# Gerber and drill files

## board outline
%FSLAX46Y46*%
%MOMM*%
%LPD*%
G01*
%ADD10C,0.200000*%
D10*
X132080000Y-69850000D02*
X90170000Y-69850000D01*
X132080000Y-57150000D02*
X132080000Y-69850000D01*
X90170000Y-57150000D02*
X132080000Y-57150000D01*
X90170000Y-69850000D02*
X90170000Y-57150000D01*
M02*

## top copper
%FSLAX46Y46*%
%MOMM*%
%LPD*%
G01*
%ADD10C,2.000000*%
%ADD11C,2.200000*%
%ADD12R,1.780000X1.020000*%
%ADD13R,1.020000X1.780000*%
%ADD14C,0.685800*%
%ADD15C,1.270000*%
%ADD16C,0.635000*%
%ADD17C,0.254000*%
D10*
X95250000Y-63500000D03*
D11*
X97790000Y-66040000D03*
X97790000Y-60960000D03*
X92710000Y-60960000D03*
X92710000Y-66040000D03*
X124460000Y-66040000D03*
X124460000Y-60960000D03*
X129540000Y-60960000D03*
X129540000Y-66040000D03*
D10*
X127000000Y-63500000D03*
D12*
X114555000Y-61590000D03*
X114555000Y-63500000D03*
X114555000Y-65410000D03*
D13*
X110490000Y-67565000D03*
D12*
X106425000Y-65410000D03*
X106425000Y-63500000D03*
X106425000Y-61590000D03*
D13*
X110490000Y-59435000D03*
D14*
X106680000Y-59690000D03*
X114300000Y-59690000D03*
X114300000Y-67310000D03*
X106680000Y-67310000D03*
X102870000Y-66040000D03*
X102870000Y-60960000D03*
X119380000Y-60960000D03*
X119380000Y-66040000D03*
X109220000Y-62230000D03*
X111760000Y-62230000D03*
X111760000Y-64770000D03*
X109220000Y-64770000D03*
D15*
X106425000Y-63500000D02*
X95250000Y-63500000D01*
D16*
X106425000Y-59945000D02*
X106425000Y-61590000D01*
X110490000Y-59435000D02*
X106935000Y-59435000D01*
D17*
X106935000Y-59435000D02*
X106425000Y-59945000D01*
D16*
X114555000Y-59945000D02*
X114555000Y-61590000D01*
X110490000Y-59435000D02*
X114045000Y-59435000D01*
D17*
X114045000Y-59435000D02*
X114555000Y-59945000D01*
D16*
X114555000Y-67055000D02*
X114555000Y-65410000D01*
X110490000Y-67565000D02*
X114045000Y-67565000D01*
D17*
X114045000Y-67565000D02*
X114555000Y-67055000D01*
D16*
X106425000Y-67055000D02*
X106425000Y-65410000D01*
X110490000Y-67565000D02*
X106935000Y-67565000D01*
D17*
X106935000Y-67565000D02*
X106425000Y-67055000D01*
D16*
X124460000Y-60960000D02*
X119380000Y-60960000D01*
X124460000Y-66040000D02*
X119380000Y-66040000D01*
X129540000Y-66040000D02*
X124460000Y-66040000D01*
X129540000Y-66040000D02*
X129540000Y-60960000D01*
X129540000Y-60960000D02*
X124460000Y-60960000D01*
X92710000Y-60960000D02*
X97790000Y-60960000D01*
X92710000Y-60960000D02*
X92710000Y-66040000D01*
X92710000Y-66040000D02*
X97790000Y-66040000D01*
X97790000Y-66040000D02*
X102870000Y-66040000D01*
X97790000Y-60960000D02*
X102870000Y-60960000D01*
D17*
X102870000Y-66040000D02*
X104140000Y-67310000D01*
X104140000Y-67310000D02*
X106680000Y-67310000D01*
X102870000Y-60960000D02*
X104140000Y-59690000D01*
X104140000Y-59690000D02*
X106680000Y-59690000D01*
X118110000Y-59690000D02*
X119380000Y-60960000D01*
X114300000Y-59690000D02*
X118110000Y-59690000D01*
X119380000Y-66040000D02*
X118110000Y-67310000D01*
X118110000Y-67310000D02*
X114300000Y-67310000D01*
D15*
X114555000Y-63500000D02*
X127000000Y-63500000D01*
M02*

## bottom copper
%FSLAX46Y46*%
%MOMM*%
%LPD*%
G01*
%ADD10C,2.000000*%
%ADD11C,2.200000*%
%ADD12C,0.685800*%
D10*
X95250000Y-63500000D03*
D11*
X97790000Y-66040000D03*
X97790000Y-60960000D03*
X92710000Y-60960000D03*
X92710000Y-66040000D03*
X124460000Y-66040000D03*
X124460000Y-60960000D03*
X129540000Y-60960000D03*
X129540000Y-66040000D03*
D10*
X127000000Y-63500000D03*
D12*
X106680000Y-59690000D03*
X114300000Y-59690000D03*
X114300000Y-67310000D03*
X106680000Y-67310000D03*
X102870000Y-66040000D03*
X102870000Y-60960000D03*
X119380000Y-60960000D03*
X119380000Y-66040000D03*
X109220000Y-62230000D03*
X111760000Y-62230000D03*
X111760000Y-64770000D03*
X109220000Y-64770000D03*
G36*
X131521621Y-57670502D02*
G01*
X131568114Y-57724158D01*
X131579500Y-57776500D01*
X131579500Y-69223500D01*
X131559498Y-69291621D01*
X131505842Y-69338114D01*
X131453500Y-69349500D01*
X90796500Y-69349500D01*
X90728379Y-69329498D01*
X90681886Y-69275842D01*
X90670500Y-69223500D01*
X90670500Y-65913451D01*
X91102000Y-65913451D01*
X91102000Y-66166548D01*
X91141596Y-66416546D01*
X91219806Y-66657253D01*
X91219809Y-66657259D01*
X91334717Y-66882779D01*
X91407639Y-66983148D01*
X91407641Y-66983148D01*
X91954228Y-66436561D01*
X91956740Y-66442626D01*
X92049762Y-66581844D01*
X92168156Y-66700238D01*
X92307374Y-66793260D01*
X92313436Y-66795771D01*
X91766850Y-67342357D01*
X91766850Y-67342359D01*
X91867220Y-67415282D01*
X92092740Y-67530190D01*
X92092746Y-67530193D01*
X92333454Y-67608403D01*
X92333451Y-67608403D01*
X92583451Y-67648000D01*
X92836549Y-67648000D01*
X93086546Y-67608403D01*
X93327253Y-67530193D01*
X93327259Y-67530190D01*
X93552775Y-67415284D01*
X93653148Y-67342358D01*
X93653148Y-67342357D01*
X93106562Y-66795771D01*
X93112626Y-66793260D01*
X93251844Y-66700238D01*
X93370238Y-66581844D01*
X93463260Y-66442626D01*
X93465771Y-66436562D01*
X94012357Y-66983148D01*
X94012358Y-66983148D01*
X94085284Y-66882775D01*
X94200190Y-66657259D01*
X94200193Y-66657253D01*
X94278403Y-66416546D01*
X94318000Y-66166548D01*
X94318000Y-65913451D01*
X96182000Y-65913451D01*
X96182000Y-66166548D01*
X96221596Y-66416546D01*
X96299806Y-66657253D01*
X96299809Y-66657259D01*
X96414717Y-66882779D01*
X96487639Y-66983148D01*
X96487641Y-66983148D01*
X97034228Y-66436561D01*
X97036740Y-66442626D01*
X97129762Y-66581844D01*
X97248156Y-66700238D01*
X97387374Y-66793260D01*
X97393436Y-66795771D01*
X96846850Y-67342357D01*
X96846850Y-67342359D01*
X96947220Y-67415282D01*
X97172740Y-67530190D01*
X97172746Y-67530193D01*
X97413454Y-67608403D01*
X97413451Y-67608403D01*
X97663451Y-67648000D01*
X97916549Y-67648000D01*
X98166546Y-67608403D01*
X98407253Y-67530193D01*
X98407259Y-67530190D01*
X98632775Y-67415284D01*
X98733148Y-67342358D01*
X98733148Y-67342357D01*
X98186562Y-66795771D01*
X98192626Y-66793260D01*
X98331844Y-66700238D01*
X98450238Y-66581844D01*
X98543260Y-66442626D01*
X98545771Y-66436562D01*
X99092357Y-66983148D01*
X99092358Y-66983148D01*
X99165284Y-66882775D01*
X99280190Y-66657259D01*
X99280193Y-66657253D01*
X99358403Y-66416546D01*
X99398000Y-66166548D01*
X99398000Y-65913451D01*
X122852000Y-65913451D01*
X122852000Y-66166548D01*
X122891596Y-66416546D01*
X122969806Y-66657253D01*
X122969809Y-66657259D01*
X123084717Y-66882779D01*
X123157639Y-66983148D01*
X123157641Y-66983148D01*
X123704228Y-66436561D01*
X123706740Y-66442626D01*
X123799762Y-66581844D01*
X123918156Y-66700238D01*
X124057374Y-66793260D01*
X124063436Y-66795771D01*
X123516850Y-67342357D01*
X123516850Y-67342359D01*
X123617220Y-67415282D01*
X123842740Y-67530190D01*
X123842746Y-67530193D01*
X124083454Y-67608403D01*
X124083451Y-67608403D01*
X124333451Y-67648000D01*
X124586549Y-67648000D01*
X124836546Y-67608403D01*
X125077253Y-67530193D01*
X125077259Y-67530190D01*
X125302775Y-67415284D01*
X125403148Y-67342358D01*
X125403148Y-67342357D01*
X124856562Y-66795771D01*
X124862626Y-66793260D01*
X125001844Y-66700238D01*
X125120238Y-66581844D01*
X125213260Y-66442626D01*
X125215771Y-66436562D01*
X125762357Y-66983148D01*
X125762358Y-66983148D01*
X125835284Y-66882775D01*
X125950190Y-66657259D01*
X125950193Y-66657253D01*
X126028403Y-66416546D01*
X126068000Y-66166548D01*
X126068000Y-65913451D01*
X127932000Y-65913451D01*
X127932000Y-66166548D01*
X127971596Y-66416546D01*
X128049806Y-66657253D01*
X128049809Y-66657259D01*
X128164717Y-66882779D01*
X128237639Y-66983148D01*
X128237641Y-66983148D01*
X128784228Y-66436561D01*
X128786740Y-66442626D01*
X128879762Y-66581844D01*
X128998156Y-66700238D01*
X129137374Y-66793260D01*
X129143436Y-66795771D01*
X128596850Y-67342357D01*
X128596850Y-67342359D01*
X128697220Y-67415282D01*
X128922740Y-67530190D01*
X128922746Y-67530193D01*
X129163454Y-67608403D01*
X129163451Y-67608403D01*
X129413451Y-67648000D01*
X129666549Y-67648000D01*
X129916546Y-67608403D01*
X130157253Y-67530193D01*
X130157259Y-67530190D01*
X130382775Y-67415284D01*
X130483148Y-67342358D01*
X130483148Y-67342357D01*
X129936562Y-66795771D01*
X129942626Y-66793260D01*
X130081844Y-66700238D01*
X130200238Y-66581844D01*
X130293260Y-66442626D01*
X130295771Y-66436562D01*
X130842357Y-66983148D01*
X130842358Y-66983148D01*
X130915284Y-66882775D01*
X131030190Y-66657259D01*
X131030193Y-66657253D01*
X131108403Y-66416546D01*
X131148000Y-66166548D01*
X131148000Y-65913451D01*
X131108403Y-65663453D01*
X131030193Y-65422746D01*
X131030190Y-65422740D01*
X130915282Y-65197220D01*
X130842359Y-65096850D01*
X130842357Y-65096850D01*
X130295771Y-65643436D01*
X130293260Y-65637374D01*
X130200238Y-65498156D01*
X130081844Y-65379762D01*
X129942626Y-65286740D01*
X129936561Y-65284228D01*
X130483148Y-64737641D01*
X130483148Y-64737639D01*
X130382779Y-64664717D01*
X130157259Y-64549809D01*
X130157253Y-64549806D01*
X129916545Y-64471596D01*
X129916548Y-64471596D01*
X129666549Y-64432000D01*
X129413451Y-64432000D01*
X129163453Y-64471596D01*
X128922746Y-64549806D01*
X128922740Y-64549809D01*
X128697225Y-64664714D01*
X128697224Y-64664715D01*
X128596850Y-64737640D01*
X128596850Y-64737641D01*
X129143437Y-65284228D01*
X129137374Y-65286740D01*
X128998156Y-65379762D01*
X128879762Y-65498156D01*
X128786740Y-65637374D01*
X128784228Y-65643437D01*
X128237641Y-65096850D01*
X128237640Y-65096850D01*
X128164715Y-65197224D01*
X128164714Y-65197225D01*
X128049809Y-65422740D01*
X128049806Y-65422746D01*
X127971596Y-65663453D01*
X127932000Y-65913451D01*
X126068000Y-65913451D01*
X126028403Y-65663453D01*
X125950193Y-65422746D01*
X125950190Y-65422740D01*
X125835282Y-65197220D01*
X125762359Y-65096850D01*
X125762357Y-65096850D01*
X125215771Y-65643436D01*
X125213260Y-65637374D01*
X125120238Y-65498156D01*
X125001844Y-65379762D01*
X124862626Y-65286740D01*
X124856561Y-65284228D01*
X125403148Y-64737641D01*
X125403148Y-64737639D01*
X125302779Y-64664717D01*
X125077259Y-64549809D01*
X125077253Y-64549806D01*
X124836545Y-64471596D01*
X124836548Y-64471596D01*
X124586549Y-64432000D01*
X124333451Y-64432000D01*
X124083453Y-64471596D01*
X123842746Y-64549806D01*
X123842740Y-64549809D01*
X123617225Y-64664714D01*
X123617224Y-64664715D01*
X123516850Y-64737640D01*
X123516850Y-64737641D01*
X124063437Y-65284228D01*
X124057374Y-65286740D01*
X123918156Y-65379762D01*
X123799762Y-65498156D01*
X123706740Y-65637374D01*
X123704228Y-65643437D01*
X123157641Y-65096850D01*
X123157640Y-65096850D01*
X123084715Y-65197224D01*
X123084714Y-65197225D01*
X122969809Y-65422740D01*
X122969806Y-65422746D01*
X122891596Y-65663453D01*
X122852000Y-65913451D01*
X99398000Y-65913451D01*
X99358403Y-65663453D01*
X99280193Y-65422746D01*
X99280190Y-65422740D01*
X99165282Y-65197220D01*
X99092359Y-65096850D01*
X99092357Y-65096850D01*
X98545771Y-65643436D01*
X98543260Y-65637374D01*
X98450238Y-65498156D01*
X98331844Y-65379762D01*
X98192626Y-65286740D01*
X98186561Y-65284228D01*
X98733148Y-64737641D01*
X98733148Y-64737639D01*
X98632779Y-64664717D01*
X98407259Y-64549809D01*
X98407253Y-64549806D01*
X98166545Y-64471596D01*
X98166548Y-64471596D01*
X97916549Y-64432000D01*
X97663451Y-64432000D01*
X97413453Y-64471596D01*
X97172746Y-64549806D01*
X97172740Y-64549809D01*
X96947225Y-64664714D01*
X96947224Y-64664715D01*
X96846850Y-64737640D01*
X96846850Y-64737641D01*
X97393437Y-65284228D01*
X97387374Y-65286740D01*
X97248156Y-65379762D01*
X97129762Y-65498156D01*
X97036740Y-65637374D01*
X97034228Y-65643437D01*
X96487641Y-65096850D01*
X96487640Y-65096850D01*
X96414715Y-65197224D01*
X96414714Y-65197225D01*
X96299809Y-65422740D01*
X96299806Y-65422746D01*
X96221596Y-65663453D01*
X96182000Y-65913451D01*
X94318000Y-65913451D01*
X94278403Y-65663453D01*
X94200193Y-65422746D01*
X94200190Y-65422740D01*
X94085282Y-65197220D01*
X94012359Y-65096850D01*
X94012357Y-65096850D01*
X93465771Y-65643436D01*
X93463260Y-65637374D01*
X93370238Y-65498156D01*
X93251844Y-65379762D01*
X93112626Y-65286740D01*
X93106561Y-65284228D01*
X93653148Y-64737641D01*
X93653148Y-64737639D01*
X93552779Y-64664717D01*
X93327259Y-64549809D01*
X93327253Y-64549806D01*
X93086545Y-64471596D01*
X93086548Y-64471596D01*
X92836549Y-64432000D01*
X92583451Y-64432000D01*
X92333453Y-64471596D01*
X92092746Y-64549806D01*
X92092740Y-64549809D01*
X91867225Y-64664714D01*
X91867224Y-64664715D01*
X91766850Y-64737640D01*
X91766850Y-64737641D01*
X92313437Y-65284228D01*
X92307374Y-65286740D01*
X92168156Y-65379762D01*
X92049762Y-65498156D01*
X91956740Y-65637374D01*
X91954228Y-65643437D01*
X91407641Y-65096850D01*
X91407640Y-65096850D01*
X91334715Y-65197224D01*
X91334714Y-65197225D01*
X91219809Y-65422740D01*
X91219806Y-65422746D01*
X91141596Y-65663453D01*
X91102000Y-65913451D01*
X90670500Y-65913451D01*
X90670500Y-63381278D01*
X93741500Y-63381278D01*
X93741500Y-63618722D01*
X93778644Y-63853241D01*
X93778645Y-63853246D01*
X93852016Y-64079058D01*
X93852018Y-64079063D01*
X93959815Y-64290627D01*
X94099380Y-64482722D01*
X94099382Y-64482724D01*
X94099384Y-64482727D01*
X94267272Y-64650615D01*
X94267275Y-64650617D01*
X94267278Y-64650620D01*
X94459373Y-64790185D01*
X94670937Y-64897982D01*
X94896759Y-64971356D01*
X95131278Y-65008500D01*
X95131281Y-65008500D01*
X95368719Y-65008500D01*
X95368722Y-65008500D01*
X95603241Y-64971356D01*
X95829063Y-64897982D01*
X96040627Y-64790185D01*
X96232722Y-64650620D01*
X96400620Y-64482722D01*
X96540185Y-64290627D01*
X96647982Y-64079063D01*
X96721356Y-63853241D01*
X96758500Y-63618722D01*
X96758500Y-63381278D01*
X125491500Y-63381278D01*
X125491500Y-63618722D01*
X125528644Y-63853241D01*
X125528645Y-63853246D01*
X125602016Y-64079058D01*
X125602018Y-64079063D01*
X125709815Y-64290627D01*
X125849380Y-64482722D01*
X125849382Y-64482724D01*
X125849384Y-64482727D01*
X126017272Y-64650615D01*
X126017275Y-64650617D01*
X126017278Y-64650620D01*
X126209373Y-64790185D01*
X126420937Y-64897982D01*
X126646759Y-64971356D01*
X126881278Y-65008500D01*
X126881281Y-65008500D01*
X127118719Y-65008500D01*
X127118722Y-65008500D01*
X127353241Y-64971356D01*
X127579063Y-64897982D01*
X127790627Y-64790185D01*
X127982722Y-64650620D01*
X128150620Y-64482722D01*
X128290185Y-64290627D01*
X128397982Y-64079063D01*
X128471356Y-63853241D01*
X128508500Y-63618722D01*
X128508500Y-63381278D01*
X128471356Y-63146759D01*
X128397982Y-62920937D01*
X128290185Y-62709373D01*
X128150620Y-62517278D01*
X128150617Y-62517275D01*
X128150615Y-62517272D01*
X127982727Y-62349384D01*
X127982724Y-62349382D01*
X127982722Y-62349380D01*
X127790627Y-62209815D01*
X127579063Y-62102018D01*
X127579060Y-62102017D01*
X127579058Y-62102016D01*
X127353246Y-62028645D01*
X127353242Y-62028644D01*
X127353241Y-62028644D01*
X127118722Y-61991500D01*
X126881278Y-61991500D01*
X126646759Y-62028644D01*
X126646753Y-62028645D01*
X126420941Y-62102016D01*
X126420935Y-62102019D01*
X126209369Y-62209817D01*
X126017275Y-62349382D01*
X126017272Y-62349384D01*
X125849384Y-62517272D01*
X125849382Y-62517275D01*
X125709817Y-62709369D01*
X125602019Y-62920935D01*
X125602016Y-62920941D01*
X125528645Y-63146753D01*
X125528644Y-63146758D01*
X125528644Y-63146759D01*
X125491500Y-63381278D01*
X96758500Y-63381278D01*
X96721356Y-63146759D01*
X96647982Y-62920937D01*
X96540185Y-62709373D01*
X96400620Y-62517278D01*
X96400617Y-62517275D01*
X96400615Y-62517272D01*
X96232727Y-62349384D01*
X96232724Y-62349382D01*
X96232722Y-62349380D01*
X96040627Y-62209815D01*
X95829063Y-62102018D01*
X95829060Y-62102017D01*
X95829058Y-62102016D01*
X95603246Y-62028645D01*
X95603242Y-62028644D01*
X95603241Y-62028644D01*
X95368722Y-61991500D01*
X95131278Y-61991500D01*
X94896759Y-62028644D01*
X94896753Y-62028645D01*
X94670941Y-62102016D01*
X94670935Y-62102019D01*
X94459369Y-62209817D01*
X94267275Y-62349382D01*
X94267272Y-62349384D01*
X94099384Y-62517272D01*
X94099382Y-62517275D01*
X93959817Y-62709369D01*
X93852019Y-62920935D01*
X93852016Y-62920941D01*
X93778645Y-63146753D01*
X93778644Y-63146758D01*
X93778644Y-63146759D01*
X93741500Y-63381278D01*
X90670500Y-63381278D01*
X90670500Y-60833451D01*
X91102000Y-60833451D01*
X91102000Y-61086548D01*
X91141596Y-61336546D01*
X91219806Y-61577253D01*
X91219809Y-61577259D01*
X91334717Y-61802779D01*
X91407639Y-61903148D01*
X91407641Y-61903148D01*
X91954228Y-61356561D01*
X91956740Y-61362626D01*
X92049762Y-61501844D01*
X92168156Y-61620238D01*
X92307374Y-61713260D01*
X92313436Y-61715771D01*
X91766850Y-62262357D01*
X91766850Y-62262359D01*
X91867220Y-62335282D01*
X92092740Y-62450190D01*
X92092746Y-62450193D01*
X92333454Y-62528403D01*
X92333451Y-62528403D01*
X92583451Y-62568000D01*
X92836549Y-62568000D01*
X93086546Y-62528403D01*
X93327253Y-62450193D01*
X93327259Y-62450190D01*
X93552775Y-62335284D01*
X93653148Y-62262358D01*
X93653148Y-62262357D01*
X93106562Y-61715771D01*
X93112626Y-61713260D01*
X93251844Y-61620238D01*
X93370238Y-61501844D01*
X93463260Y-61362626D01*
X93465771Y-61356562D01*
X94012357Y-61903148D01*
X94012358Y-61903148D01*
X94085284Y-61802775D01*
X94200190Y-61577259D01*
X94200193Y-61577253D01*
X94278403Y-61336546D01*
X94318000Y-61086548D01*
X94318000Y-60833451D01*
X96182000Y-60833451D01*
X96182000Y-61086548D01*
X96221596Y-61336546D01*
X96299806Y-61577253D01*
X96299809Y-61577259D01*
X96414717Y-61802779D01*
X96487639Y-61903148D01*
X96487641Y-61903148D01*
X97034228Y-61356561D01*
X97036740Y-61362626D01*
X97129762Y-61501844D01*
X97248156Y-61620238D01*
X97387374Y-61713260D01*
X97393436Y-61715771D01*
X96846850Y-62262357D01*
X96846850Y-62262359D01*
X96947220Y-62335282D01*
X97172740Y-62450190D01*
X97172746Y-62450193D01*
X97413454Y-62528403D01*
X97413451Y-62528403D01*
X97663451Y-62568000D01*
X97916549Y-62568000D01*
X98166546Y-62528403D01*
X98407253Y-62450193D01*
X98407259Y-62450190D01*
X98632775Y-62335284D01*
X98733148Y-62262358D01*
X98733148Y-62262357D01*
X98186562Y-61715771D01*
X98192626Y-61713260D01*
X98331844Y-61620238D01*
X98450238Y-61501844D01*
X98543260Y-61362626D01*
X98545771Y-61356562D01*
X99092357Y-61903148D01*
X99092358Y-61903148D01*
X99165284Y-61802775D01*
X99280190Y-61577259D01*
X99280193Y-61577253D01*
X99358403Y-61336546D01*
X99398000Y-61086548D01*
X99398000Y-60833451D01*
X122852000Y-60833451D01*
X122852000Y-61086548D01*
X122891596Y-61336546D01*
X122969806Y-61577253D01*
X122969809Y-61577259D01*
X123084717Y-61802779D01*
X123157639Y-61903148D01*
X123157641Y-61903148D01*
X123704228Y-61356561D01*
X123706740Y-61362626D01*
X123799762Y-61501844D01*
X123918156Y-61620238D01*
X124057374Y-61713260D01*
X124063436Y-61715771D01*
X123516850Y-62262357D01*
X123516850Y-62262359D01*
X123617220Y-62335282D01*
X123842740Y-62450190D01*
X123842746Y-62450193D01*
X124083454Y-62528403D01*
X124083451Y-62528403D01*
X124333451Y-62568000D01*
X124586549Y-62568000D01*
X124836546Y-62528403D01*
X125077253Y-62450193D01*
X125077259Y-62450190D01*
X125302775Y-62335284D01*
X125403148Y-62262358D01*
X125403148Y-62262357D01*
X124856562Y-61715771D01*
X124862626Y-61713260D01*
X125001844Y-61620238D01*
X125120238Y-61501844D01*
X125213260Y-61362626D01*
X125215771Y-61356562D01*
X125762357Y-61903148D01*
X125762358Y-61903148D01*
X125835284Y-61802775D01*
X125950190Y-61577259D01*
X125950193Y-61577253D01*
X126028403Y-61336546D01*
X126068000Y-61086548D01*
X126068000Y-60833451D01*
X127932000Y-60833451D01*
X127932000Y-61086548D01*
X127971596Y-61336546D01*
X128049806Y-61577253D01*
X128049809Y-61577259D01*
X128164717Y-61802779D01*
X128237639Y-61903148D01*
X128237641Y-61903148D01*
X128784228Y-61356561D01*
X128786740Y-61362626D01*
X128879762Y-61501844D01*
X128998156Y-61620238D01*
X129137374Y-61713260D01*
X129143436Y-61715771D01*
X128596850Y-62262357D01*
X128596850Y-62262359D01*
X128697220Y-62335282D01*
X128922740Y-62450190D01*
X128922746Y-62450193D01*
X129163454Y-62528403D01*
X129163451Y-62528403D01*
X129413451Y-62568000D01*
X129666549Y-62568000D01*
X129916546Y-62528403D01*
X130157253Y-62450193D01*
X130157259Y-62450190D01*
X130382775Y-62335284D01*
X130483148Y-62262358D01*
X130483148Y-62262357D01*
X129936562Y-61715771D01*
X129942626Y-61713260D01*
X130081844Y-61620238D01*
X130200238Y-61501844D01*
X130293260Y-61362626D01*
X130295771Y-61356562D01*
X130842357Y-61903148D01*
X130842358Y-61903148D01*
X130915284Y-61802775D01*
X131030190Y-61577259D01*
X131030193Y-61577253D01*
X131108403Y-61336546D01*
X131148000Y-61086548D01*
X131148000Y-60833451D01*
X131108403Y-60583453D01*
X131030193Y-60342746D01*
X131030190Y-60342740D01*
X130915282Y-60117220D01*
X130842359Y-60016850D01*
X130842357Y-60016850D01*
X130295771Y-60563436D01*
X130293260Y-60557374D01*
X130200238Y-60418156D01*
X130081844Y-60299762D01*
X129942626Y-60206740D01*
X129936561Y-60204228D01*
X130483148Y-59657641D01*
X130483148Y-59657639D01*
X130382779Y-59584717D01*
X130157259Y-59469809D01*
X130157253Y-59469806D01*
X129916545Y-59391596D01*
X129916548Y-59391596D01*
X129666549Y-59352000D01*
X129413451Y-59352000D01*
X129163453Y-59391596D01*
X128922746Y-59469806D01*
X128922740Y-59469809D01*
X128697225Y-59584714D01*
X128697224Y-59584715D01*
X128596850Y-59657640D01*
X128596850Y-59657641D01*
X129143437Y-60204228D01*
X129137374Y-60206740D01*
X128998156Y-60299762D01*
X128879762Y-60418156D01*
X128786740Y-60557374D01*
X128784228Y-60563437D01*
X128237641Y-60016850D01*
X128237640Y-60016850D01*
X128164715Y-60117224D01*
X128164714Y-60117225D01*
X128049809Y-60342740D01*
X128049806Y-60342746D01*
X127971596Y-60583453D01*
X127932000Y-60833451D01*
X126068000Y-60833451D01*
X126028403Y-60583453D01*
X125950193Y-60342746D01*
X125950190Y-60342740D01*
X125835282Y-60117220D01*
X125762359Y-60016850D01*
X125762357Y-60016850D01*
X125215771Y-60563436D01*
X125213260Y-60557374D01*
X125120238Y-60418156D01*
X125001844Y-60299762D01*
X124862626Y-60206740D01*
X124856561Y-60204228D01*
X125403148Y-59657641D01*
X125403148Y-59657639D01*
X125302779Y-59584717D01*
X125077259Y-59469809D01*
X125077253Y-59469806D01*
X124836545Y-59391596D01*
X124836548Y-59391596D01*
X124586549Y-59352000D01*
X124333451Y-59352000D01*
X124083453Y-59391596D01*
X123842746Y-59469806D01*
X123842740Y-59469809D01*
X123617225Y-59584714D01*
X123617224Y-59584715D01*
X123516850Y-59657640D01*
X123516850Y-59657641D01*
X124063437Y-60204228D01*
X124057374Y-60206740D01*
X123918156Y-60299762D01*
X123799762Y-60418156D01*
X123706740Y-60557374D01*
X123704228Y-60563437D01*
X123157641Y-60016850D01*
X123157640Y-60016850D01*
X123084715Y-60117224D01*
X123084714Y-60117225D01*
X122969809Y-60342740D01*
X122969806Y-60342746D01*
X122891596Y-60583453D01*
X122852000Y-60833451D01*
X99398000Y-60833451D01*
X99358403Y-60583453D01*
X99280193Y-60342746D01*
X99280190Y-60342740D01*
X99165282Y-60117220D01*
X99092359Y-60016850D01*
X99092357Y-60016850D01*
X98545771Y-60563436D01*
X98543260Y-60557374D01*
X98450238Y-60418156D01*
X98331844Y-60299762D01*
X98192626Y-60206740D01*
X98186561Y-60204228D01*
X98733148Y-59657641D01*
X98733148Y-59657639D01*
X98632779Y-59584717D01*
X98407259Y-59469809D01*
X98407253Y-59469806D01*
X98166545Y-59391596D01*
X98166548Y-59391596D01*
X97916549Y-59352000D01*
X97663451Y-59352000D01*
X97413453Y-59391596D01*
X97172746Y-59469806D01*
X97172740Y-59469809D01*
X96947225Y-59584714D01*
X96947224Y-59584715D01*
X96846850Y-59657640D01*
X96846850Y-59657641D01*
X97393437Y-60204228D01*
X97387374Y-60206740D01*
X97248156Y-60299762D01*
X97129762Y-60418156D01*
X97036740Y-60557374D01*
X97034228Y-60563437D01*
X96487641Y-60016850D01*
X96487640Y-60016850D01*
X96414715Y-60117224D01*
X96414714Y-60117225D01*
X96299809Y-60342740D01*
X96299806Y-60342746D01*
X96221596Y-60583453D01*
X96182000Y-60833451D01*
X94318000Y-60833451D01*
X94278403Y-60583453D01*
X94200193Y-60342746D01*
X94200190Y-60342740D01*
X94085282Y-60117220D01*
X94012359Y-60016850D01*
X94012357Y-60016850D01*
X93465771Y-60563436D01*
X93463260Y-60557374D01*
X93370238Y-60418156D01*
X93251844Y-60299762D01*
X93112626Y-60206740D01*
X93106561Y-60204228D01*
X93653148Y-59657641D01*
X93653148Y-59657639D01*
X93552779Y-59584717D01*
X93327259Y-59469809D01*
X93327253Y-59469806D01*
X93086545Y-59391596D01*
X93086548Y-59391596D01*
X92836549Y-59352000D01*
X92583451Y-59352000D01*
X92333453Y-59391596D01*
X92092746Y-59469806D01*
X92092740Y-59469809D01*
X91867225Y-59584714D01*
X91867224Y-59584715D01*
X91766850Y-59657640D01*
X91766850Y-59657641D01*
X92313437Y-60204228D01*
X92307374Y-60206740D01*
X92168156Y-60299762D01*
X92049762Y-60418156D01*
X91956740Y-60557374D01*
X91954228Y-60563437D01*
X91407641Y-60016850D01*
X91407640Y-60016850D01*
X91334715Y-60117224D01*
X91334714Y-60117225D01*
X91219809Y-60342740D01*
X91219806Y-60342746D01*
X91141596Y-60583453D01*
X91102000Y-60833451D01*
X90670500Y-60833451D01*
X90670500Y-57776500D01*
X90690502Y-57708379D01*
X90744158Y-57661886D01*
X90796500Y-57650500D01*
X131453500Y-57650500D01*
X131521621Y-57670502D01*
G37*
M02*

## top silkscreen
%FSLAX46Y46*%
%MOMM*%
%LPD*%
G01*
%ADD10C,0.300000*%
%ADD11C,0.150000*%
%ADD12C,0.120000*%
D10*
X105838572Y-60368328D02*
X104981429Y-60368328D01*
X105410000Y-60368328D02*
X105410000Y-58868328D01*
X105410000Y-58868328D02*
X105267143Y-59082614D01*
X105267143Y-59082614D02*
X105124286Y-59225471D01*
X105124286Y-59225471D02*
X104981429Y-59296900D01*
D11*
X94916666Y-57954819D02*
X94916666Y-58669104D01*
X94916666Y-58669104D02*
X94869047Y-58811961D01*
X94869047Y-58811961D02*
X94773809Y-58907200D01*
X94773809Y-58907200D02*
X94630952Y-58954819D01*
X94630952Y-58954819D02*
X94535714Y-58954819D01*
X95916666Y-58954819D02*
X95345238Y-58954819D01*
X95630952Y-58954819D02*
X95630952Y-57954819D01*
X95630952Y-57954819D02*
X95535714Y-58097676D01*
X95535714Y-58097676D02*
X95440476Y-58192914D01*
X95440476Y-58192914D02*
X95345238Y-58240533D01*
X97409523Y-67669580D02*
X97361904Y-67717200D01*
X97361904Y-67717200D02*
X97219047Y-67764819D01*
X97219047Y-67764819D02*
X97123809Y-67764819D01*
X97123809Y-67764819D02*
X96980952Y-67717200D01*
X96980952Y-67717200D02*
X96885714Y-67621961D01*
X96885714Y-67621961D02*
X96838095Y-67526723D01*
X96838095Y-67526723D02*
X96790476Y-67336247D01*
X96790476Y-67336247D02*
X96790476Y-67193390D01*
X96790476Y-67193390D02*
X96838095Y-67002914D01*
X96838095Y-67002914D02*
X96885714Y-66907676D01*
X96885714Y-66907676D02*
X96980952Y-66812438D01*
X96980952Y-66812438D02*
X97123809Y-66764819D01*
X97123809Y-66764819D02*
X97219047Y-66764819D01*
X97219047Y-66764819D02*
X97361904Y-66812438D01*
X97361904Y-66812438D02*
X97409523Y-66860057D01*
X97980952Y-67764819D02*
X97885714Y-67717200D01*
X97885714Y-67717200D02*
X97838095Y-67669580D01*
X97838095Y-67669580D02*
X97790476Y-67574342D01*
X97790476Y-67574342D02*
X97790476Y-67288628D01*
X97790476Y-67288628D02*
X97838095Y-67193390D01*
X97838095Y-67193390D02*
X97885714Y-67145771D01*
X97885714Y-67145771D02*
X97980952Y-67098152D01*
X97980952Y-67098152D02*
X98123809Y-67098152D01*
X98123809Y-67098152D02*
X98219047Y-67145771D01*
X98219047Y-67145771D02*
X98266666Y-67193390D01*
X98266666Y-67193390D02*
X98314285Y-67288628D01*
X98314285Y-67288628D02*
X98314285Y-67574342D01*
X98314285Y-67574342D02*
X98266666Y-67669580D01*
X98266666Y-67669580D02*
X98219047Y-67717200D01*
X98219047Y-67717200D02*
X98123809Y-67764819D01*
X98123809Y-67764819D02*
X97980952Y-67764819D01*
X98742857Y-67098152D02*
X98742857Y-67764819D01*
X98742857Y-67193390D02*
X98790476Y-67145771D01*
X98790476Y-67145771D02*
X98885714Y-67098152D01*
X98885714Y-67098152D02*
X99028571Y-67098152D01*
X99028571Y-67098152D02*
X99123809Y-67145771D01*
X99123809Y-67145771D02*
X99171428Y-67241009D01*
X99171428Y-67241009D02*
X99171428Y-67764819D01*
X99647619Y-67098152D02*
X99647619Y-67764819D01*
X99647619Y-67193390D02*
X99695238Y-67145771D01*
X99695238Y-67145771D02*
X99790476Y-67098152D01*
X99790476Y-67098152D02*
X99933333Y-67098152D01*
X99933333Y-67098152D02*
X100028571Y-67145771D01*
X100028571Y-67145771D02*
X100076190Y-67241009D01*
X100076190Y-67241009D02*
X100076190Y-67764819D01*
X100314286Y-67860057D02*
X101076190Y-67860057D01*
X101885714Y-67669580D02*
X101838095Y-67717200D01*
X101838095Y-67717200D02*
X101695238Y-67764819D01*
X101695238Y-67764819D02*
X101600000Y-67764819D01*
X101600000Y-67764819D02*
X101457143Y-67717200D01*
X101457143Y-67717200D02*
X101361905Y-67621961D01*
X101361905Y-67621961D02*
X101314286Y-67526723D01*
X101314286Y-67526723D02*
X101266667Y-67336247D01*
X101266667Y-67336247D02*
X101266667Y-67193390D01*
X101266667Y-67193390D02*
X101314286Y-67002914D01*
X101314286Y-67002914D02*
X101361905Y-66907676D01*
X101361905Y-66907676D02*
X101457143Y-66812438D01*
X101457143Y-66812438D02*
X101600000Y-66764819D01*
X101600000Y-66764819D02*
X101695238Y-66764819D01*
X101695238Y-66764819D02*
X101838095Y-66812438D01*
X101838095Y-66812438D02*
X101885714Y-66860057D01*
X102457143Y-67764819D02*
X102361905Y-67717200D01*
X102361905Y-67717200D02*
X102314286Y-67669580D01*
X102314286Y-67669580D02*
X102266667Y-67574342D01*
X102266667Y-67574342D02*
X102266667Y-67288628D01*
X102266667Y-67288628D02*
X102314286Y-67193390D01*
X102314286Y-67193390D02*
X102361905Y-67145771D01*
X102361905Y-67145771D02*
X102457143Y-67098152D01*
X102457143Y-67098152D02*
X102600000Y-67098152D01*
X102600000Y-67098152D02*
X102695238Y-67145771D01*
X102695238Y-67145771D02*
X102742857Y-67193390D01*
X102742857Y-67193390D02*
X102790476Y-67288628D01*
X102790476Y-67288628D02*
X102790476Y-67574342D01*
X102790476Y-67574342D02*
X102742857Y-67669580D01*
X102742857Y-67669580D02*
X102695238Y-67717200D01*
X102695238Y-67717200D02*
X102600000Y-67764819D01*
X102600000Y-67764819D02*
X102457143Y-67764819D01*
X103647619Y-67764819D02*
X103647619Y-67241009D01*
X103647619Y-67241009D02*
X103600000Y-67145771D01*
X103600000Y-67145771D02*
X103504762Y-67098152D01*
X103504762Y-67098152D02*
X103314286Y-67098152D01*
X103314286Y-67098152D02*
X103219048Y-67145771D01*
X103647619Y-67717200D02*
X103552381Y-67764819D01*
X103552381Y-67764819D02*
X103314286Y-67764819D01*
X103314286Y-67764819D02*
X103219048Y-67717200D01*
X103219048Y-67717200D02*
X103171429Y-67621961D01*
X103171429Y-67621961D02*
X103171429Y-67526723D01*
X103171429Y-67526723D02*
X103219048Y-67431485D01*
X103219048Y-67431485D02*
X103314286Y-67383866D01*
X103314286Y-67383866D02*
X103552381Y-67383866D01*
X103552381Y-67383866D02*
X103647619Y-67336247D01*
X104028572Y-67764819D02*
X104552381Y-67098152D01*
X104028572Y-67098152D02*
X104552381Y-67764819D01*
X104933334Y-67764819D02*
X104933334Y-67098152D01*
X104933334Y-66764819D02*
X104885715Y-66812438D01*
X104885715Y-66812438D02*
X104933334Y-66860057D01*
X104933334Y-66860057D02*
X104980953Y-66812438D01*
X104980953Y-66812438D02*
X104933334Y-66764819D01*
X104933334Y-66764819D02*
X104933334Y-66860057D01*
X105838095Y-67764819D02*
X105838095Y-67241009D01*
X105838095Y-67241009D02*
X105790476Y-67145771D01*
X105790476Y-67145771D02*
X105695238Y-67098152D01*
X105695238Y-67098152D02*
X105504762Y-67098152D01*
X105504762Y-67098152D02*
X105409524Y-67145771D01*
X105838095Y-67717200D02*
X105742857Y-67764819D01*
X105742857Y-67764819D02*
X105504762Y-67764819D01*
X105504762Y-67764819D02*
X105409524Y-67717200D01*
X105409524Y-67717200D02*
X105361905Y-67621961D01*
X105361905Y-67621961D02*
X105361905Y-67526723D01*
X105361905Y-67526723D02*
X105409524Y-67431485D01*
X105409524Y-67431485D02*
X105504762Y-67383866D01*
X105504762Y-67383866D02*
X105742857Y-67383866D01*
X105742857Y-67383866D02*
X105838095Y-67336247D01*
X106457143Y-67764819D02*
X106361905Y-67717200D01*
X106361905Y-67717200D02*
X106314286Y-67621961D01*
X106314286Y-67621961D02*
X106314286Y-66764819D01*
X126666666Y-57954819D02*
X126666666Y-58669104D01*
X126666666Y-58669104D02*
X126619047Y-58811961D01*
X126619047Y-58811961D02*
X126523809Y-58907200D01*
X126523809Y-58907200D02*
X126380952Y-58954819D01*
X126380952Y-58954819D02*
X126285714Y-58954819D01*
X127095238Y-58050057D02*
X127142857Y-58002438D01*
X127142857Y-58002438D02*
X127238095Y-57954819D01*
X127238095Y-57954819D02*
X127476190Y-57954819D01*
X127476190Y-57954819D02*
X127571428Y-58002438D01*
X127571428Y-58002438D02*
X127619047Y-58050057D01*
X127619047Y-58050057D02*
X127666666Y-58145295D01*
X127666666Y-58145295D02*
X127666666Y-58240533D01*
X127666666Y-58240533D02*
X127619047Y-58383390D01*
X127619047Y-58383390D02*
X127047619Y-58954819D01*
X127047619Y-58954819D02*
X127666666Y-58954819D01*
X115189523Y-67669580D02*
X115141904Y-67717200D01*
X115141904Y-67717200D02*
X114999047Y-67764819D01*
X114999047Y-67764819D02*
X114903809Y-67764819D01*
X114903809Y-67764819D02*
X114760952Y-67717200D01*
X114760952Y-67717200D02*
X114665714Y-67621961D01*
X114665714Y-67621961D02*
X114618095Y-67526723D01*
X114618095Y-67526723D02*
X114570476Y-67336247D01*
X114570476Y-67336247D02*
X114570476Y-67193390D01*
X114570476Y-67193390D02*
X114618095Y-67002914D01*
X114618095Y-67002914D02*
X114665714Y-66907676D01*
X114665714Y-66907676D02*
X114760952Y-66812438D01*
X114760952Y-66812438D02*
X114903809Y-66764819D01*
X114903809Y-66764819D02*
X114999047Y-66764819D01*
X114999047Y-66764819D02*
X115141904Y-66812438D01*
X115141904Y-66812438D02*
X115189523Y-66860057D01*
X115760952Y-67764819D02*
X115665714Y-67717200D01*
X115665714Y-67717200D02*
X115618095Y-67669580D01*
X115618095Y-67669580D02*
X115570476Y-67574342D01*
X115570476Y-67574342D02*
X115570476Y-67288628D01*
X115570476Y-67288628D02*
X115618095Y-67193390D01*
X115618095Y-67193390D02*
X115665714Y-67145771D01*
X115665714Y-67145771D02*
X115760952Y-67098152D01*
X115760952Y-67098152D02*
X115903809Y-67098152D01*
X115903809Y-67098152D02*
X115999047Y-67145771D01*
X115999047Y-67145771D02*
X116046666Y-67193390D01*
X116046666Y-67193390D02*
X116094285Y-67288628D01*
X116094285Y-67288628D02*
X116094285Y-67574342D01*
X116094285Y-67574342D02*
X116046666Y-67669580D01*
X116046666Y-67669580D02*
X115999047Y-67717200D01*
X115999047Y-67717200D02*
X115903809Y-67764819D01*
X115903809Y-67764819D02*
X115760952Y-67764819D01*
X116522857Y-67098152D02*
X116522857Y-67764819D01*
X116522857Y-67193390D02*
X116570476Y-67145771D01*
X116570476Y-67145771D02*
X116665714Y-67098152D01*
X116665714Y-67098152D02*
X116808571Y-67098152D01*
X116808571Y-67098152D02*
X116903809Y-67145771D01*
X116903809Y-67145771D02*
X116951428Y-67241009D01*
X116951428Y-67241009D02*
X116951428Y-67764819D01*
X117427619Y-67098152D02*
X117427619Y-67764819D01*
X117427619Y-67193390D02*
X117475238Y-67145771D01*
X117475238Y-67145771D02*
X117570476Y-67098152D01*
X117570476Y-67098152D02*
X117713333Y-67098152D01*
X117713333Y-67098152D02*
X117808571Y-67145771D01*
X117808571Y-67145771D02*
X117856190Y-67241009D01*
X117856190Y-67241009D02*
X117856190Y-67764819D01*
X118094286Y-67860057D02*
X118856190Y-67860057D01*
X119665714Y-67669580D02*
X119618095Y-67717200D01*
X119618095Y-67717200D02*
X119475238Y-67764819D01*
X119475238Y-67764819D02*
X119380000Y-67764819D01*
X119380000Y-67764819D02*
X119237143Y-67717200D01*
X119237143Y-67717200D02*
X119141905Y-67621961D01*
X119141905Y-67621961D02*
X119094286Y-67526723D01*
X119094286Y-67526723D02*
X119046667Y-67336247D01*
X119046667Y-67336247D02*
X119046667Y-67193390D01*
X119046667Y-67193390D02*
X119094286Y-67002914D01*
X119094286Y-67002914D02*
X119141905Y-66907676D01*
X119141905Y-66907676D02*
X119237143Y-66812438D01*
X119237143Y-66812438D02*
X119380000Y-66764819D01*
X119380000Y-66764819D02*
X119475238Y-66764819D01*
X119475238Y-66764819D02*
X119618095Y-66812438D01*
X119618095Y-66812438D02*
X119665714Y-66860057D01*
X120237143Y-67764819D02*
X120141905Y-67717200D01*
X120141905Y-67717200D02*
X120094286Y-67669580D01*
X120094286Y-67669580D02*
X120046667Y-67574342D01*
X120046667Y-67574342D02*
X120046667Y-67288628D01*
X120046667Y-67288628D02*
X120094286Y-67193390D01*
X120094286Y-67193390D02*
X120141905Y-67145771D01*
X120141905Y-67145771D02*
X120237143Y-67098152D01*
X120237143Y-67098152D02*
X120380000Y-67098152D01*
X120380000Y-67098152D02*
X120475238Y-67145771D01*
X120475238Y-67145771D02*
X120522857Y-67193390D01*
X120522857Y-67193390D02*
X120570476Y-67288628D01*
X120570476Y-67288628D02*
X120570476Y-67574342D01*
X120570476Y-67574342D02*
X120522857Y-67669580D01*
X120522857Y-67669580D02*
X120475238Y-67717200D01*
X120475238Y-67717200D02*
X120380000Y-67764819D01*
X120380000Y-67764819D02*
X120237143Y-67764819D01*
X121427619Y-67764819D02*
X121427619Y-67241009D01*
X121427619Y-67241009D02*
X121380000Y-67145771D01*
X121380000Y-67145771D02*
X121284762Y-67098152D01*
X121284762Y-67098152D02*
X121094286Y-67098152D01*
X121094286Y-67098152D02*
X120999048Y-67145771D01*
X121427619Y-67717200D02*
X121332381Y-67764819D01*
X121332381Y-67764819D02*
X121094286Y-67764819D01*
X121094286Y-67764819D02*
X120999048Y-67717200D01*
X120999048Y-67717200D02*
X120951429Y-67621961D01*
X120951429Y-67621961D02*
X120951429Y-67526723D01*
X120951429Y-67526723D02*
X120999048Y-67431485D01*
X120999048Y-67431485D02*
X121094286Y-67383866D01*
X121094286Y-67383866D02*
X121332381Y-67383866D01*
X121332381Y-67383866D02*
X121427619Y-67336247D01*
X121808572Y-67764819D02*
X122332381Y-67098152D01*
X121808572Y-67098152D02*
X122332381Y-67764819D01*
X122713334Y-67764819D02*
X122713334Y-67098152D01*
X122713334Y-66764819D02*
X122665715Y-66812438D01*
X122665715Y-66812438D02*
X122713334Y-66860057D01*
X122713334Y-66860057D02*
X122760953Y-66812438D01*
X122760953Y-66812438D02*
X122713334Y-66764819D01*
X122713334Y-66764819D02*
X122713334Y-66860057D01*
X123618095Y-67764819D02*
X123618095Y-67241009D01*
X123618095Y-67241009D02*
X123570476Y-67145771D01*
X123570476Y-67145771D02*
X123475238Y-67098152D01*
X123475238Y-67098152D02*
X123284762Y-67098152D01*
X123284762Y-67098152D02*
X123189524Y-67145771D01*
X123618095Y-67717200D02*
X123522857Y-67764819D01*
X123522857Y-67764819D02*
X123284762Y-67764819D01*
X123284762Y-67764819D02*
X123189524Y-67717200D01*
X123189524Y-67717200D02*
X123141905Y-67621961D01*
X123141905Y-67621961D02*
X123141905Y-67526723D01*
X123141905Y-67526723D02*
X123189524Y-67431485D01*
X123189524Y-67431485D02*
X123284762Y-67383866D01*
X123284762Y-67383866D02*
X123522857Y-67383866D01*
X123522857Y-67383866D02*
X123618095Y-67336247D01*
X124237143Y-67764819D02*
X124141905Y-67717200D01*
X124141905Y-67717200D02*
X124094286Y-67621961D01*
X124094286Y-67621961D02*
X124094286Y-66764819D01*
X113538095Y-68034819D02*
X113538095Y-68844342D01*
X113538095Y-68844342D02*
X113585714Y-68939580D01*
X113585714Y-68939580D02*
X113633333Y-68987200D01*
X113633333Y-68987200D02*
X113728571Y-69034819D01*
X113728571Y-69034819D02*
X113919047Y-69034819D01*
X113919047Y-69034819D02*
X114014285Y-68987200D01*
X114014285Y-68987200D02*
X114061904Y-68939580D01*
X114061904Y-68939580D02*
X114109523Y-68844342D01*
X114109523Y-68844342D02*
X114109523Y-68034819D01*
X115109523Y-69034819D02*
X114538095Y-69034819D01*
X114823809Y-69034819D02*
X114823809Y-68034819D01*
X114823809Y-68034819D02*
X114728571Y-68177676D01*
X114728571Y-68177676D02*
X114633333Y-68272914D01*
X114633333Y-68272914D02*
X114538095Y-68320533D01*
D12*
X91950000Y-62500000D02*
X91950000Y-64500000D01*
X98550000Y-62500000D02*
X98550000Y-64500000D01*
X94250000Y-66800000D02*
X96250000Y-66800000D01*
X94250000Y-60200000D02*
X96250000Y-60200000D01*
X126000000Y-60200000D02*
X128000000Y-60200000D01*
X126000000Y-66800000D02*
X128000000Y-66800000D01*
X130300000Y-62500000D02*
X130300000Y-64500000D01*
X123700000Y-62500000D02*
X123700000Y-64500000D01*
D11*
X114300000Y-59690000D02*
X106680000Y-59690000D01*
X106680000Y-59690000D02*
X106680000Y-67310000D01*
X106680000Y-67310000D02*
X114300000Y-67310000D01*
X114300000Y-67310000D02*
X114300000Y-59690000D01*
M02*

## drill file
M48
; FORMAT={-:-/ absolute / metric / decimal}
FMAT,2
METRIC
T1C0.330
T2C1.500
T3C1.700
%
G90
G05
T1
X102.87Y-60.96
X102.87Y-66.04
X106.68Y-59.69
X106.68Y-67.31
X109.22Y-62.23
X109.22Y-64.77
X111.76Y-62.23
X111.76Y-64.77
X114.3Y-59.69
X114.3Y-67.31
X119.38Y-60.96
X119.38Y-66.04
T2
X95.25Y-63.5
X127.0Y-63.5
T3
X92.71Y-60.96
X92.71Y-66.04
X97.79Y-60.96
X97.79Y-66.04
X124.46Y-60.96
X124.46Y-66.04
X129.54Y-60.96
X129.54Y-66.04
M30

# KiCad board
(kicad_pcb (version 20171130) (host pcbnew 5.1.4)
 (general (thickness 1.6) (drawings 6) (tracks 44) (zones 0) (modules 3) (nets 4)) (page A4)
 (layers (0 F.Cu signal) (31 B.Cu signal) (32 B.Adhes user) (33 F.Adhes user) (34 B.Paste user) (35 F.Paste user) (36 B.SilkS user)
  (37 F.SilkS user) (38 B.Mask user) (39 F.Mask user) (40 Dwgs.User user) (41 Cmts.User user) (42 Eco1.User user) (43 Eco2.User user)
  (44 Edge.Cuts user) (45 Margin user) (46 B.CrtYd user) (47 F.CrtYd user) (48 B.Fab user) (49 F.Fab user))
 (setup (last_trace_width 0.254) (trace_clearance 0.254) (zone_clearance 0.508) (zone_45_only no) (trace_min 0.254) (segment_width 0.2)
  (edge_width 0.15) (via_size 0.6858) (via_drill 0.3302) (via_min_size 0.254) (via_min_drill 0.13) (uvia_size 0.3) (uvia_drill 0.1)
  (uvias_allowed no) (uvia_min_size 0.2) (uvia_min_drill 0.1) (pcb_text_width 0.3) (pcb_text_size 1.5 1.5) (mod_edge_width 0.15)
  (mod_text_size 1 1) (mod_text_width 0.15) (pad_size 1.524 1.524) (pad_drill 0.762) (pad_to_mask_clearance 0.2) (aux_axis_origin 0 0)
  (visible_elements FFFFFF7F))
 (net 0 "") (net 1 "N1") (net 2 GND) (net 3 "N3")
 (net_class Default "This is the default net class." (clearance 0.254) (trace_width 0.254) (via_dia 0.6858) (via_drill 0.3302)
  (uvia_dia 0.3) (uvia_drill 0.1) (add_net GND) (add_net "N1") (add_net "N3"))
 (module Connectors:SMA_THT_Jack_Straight (layer F.Cu) (at 95.25 63.5)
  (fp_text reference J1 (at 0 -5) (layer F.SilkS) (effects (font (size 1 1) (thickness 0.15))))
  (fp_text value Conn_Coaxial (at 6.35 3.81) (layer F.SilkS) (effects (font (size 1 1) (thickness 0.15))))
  (fp_line (start -3.3 -1) (end -3.3 1) (layer F.SilkS) (width 0.12))
  (fp_line (start 3.3 -1) (end 3.3 1) (layer F.SilkS) (width 0.12))
  (fp_line (start -1 3.3) (end 1 3.3) (layer F.SilkS) (width 0.12))
  (fp_line (start -1 -3.3) (end 1 -3.3) (layer F.SilkS) (width 0.12))
  (pad 1 thru_hole circle (at 0 0) (size 2 2) (drill 1.5) (layers *.Cu *.Mask) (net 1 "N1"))
  (pad 2 thru_hole circle (at 2.54 2.54) (size 2.2 2.2) (drill 1.7) (layers *.Cu *.Mask) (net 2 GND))
  (pad 2 thru_hole circle (at 2.54 -2.54) (size 2.2 2.2) (drill 1.7) (layers *.Cu *.Mask) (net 2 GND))
  (pad 2 thru_hole circle (at -2.54 -2.54) (size 2.2 2.2) (drill 1.7) (layers *.Cu *.Mask) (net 2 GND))
  (pad 2 thru_hole circle (at -2.54 2.54) (size 2.2 2.2) (drill 1.7) (layers *.Cu *.Mask) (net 2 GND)))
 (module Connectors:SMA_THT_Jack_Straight (layer F.Cu) (at 127 63.5)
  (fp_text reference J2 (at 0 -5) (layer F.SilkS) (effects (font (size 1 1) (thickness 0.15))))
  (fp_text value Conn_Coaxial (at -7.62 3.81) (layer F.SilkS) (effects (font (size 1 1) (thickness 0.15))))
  (fp_line (start -1 -3.3) (end 1 -3.3) (layer F.SilkS) (width 0.12))
  (fp_line (start -1 3.3) (end 1 3.3) (layer F.SilkS) (width 0.12))
  (fp_line (start 3.3 -1) (end 3.3 1) (layer F.SilkS) (width 0.12))
  (fp_line (start -3.3 -1) (end -3.3 1) (layer F.SilkS) (width 0.12))
  (pad 2 thru_hole circle (at -2.54 2.54) (size 2.2 2.2) (drill 1.7) (layers *.Cu *.Mask) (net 2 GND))
  (pad 2 thru_hole circle (at -2.54 -2.54) (size 2.2 2.2) (drill 1.7) (layers *.Cu *.Mask) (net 2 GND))
  (pad 2 thru_hole circle (at 2.54 -2.54) (size 2.2 2.2) (drill 1.7) (layers *.Cu *.Mask) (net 2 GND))
  (pad 2 thru_hole circle (at 2.54 2.54) (size 2.2 2.2) (drill 1.7) (layers *.Cu *.Mask) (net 2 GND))
  (pad 1 thru_hole circle (at 0 0) (size 2 2) (drill 1.5) (layers *.Cu *.Mask) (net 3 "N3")))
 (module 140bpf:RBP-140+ (layer F.Cu) (at 110.49 63.5 270)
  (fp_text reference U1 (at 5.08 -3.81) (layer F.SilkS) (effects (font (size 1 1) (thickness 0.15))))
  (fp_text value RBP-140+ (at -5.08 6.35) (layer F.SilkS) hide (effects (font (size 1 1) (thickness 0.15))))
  (fp_line (start -3.81 -3.81) (end -3.81 3.81) (layer F.SilkS) (width 0.15))
  (fp_line (start -3.81 3.81) (end 3.81 3.81) (layer F.SilkS) (width 0.15))
  (fp_line (start 3.81 3.81) (end 3.81 -3.81) (layer F.SilkS) (width 0.15))
  (fp_line (start 3.81 -3.81) (end -3.81 -3.81) (layer F.SilkS) (width 0.15))
  (pad 7 smd rect (at -1.91 -4.065 270) (size 1.02 1.78) (layers F.Cu F.Paste F.Mask) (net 2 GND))
  (pad 6 smd rect (at 0 -4.065 270) (size 1.02 1.78) (layers F.Cu F.Paste F.Mask) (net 3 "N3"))
  (pad 5 smd rect (at 1.91 -4.065 270) (size 1.02 1.78) (layers F.Cu F.Paste F.Mask) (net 2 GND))
  (pad 4 smd rect (at 4.065 0) (size 1.02 1.78) (layers F.Cu F.Paste F.Mask) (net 2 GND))
  (pad 3 smd rect (at 1.91 4.065 90) (size 1.02 1.78) (layers F.Cu F.Paste F.Mask) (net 2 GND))
  (pad 2 smd rect (at 0 4.065 270) (size 1.02 1.78) (layers F.Cu F.Paste F.Mask) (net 1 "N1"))
  (pad 1 smd rect (at -1.91 4.065 270) (size 1.02 1.78) (layers F.Cu F.Paste F.Mask) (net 2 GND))
  (pad 8 smd rect (at -4.065 0) (size 1.02 1.78) (layers F.Cu F.Paste F.Mask) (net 2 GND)))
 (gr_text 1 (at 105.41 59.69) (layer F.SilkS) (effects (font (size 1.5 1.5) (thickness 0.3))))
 (gr_line (start 132.08 69.85) (end 90.17 69.85) (layer Edge.Cuts) (width 0.2))
 (gr_line (start 132.08 57.15) (end 132.08 69.85) (layer Edge.Cuts) (width 0.2))
 (gr_line (start 90.17 57.15) (end 132.08 57.15) (layer Edge.Cuts) (width 0.2))
 (gr_line (start 90.17 69.85) (end 90.17 57.15) (layer Edge.Cuts) (width 0.2))
 (segment (start 106.425 63.5) (end 95.25 63.5) (width 1.27) (layer F.Cu) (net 1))
 (via (at 106.68 59.69) (size 0.6858) (drill 0.3302) (layers F.Cu B.Cu) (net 2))
 (via (at 114.3 59.69) (size 0.6858) (drill 0.3302) (layers F.Cu B.Cu) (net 2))
 (via (at 114.3 67.31) (size 0.6858) (drill 0.3302) (layers F.Cu B.Cu) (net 2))
 (via (at 106.68 67.31) (size 0.6858) (drill 0.3302) (layers F.Cu B.Cu) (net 2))
 (segment (start 106.425 59.945) (end 106.425 61.59) (width 0.635) (layer F.Cu) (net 2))
 (segment (start 110.49 59.435) (end 106.935 59.435) (width 0.635) (layer F.Cu) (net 2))
 (segment (start 106.935 59.435) (end 106.425 59.945) (width 0.254) (layer F.Cu) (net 2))
 (segment (start 114.555 59.945) (end 114.555 61.59) (width 0.635) (layer F.Cu) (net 2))
 (segment (start 110.49 59.435) (end 114.045 59.435) (width 0.635) (layer F.Cu) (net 2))
 (segment (start 114.045 59.435) (end 114.555 59.945) (width 0.254) (layer F.Cu) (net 2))
 (segment (start 114.555 67.055) (end 114.555 65.41) (width 0.635) (layer F.Cu) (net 2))
 (segment (start 110.49 67.565) (end 114.045 67.565) (width 0.635) (layer F.Cu) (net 2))
 (segment (start 114.045 67.565) (end 114.555 67.055) (width 0.254) (layer F.Cu) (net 2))
 (segment (start 106.425 67.055) (end 106.425 65.41) (width 0.635) (layer F.Cu) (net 2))
 (segment (start 110.49 67.565) (end 106.935 67.565) (width 0.635) (layer F.Cu) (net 2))
 (segment (start 106.935 67.565) (end 106.425 67.055) (width 0.254) (layer F.Cu) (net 2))
 (via (at 102.87 66.04) (size 0.6858) (drill 0.3302) (layers F.Cu B.Cu) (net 2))
 (via (at 102.87 60.96) (size 0.6858) (drill 0.3302) (layers F.Cu B.Cu) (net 2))
 (via (at 119.38 60.96) (size 0.6858) (drill 0.3302) (layers F.Cu B.Cu) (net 2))
 (via (at 119.38 66.04) (size 0.6858) (drill 0.3302) (layers F.Cu B.Cu) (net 2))
 (segment (start 124.46 60.96) (end 119.38 60.96) (width 0.635) (layer F.Cu) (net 2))
 (segment (start 124.46 66.04) (end 119.38 66.04) (width 0.635) (layer F.Cu) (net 2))
 (segment (start 129.54 66.04) (end 124.46 66.04) (width 0.635) (layer F.Cu) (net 2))
 (segment (start 129.54 66.04) (end 129.54 60.96) (width 0.635) (layer F.Cu) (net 2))
 (segment (start 129.54 60.96) (end 124.46 60.96) (width 0.635) (layer F.Cu) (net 2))
 (segment (start 92.71 60.96) (end 97.79 60.96) (width 0.635) (layer F.Cu) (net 2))
 (segment (start 92.71 60.96) (end 92.71 66.04) (width 0.635) (layer F.Cu) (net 2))
 (segment (start 92.71 66.04) (end 97.79 66.04) (width 0.635) (layer F.Cu) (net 2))
 (segment (start 97.79 66.04) (end 102.87 66.04) (width 0.635) (layer F.Cu) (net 2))
 (segment (start 97.79 60.96) (end 102.87 60.96) (width 0.635) (layer F.Cu) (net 2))
 (segment (start 102.87 66.04) (end 104.14 67.31) (width 0.254) (layer F.Cu) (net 2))
 (segment (start 104.14 67.31) (end 106.68 67.31) (width 0.254) (layer F.Cu) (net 2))
 (segment (start 102.87 60.96) (end 104.14 59.69) (width 0.254) (layer F.Cu) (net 2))
 (segment (start 104.14 59.69) (end 106.68 59.69) (width 0.254) (layer F.Cu) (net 2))
 (segment (start 118.11 59.69) (end 119.38 60.96) (width 0.254) (layer F.Cu) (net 2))
 (segment (start 114.3 59.69) (end 118.11 59.69) (width 0.254) (layer F.Cu) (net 2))
 (segment (start 119.38 66.04) (end 118.11 67.31) (width 0.254) (layer F.Cu) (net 2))
 (segment (start 118.11 67.31) (end 114.3 67.31) (width 0.254) (layer F.Cu) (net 2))
 (via (at 109.22 62.23) (size 0.6858) (drill 0.3302) (layers F.Cu B.Cu) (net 2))
 (via (at 111.76 62.23) (size 0.6858) (drill 0.3302) (layers F.Cu B.Cu) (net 2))
 (via (at 111.76 64.77) (size 0.6858) (drill 0.3302) (layers F.Cu B.Cu) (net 2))
 (via (at 109.22 64.77) (size 0.6858) (drill 0.3302) (layers F.Cu B.Cu) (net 2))
 (segment (start 114.555 63.5) (end 127 63.5) (width 1.27) (layer F.Cu) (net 3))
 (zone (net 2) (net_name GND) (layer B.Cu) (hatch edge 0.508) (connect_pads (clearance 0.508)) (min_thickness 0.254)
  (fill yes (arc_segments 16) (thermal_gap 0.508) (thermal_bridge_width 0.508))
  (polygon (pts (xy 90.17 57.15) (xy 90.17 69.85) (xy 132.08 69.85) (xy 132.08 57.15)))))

